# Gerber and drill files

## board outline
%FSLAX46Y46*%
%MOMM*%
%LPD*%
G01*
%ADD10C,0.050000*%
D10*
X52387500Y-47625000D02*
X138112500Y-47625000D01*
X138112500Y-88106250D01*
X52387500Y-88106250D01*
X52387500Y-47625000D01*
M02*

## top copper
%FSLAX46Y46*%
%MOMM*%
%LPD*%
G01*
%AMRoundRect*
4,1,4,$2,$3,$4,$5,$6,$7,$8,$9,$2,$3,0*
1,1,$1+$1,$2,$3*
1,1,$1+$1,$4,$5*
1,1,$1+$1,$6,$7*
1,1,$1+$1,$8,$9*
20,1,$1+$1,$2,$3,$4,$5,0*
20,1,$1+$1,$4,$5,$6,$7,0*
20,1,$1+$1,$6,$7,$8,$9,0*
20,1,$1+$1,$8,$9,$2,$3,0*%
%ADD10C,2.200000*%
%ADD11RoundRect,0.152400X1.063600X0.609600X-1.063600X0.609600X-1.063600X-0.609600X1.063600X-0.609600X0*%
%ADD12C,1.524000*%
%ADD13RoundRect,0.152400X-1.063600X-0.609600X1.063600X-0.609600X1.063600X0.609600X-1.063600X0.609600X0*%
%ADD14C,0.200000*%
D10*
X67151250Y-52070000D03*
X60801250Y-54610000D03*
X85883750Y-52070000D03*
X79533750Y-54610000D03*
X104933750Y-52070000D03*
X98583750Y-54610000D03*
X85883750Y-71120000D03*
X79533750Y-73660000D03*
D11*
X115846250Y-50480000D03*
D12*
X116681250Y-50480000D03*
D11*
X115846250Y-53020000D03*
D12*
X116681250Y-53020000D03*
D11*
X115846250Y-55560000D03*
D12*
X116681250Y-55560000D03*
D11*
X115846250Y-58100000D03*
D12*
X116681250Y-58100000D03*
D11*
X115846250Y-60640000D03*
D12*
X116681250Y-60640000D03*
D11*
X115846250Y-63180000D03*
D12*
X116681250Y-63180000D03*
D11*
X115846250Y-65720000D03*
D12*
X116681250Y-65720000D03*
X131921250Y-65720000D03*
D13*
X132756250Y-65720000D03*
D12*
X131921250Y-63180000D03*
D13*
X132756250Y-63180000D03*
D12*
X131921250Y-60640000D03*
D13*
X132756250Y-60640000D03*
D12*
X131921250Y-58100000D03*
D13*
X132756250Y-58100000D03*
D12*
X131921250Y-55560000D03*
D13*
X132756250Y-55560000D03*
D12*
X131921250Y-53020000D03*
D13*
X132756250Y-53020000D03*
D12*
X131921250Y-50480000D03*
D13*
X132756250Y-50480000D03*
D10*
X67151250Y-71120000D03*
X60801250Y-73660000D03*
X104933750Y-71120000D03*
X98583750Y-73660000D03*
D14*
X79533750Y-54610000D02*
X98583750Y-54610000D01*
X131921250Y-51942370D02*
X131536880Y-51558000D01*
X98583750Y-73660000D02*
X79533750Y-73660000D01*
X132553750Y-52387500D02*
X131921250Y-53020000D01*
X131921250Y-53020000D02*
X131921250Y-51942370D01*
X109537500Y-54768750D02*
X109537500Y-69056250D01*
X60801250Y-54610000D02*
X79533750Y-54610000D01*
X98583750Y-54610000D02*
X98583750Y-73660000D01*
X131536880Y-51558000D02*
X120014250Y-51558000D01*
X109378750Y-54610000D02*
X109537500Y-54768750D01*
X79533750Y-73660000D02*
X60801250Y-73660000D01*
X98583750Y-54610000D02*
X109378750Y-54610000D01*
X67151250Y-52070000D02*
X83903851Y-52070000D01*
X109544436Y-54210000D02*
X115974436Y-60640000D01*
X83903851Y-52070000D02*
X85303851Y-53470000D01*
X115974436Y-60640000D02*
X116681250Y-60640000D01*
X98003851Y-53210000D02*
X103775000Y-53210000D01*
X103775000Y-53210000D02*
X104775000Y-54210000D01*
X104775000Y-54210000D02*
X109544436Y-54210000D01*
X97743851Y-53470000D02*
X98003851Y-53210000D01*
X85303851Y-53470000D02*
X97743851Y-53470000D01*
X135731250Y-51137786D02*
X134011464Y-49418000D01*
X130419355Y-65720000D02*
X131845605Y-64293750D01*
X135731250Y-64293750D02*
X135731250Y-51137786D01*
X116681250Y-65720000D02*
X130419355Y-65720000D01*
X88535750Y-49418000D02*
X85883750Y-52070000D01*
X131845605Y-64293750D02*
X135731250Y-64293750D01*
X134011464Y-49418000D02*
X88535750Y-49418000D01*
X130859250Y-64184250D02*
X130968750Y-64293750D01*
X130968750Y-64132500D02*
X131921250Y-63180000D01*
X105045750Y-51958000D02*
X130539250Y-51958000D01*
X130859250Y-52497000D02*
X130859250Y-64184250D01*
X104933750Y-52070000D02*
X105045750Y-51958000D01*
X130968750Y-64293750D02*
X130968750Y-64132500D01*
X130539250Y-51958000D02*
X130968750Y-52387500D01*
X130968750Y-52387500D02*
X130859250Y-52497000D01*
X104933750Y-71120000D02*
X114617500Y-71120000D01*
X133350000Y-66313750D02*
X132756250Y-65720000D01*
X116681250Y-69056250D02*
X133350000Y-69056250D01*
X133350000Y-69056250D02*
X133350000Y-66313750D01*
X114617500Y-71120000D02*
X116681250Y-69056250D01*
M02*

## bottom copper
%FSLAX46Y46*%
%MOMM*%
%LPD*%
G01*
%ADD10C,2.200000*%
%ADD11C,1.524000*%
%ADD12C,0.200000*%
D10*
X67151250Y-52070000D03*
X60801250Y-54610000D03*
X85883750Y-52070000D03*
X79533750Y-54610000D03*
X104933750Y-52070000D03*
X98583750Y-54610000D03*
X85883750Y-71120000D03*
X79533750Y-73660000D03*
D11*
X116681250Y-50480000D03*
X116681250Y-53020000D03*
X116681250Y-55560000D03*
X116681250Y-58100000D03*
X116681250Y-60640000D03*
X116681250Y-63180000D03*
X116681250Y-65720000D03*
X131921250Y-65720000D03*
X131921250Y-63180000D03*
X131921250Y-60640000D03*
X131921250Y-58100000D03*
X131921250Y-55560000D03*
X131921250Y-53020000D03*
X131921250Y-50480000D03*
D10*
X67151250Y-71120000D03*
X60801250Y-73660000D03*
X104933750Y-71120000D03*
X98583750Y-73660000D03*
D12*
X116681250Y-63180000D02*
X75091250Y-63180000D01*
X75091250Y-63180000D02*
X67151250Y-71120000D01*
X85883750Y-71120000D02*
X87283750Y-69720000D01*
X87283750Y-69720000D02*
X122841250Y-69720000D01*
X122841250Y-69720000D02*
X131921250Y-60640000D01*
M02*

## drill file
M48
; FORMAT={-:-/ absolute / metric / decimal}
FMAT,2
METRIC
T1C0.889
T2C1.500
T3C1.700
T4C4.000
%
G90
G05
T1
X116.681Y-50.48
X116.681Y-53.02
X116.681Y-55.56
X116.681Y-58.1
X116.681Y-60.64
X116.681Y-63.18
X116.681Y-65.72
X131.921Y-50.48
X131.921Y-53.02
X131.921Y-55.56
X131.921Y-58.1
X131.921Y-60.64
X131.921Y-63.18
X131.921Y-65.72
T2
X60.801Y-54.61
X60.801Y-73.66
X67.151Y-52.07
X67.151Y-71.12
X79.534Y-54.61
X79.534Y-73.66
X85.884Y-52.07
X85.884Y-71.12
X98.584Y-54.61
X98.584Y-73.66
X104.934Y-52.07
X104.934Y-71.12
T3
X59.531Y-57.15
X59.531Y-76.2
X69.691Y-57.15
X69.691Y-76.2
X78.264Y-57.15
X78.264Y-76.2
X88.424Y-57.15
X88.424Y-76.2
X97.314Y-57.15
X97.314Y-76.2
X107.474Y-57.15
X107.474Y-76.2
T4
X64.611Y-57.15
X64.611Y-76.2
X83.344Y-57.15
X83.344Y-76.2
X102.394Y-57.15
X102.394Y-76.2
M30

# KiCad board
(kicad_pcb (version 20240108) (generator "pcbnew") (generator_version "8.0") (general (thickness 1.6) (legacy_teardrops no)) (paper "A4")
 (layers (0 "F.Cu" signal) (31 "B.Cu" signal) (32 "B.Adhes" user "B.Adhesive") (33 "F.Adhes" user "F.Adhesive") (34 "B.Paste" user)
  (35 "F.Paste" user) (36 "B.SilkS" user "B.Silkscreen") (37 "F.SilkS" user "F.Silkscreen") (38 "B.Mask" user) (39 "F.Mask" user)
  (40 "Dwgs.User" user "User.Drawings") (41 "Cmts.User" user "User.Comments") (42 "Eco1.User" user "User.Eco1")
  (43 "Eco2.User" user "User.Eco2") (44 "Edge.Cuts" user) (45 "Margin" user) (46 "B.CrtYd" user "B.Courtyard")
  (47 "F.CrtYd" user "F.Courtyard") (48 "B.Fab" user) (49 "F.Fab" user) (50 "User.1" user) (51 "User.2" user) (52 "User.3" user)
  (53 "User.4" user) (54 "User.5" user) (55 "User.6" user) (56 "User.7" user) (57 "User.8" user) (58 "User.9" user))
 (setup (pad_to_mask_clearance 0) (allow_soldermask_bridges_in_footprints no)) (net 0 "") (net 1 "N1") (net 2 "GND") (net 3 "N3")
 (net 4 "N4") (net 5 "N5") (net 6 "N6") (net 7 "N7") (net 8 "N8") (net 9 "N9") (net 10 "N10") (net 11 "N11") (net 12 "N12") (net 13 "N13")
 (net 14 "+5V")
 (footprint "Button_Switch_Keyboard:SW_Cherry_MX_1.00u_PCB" (layer "F.Cu") (at 67.15125 52.07)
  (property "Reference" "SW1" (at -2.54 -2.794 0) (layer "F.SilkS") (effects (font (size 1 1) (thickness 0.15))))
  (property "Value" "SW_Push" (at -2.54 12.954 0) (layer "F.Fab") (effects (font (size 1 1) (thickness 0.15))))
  (pad "" np_thru_hole circle (at -7.62 5.08) (size 1.7 1.7) (drill 1.7) (layers "*.Cu" "*.Mask"))
  (pad "" np_thru_hole circle (at -2.54 5.08) (size 4 4) (drill 4) (layers "*.Cu" "*.Mask"))
  (pad "" np_thru_hole circle (at 2.54 5.08) (size 1.7 1.7) (drill 1.7) (layers "*.Cu" "*.Mask"))
  (pad "1" thru_hole circle (at 0 0) (size 2.2 2.2) (drill 1.5) (layers "*.Cu" "*.Mask") (remove_unused_layers no) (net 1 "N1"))
  (pad "2" thru_hole circle (at -6.35 2.54) (size 2.2 2.2) (drill 1.5) (layers "*.Cu" "*.Mask") (remove_unused_layers no) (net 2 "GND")))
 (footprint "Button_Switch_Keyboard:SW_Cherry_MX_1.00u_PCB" (layer "F.Cu") (at 85.88375 52.07)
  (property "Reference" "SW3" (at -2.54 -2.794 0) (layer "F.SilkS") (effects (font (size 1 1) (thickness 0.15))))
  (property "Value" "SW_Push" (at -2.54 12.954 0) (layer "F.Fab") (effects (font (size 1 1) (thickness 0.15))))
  (pad "" np_thru_hole circle (at -7.62 5.08) (size 1.7 1.7) (drill 1.7) (layers "*.Cu" "*.Mask"))
  (pad "" np_thru_hole circle (at -2.54 5.08) (size 4 4) (drill 4) (layers "*.Cu" "*.Mask"))
  (pad "" np_thru_hole circle (at 2.54 5.08) (size 1.7 1.7) (drill 1.7) (layers "*.Cu" "*.Mask"))
  (pad "1" thru_hole circle (at 0 0) (size 2.2 2.2) (drill 1.5) (layers "*.Cu" "*.Mask") (remove_unused_layers no) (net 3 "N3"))
  (pad "2" thru_hole circle (at -6.35 2.54) (size 2.2 2.2) (drill 1.5) (layers "*.Cu" "*.Mask") (remove_unused_layers no) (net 2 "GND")))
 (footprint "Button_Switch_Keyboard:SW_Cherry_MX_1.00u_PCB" (layer "F.Cu") (at 104.93375 52.07)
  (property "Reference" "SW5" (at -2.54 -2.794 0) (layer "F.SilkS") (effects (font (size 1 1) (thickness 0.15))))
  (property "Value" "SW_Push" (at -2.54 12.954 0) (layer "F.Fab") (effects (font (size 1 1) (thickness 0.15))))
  (pad "" np_thru_hole circle (at -7.62 5.08) (size 1.7 1.7) (drill 1.7) (layers "*.Cu" "*.Mask"))
  (pad "" np_thru_hole circle (at -2.54 5.08) (size 4 4) (drill 4) (layers "*.Cu" "*.Mask"))
  (pad "" np_thru_hole circle (at 2.54 5.08) (size 1.7 1.7) (drill 1.7) (layers "*.Cu" "*.Mask"))
  (pad "1" thru_hole circle (at 0 0) (size 2.2 2.2) (drill 1.5) (layers "*.Cu" "*.Mask") (remove_unused_layers no) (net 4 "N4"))
  (pad "2" thru_hole circle (at -6.35 2.54) (size 2.2 2.2) (drill 1.5) (layers "*.Cu" "*.Mask") (remove_unused_layers no) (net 2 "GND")))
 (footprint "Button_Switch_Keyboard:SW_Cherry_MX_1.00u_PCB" (layer "F.Cu") (at 85.88375 71.12)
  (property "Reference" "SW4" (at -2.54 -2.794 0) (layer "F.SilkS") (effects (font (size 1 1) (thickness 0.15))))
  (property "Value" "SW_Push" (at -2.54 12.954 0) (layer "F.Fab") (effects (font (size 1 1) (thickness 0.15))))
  (pad "" np_thru_hole circle (at -7.62 5.08) (size 1.7 1.7) (drill 1.7) (layers "*.Cu" "*.Mask"))
  (pad "" np_thru_hole circle (at -2.54 5.08) (size 4 4) (drill 4) (layers "*.Cu" "*.Mask"))
  (pad "" np_thru_hole circle (at 2.54 5.08) (size 1.7 1.7) (drill 1.7) (layers "*.Cu" "*.Mask"))
  (pad "1" thru_hole circle (at 0 0) (size 2.2 2.2) (drill 1.5) (layers "*.Cu" "*.Mask") (remove_unused_layers no) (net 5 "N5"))
  (pad "2" thru_hole circle (at -6.35 2.54) (size 2.2 2.2) (drill 1.5) (layers "*.Cu" "*.Mask") (remove_unused_layers no) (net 2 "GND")))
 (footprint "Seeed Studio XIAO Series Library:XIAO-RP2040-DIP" (layer "F.Cu") (at 124.30125 58.1)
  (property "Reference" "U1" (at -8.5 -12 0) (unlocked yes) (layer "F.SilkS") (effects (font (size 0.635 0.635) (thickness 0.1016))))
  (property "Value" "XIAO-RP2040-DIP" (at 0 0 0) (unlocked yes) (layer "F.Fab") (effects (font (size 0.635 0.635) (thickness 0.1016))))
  (pad "1" smd roundrect (at -8.455 -7.62 180) (size 2.432 1.524) (layers "F.Cu" "F.Mask") (roundrect_rratio 0.1) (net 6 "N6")
   (thermal_bridge_angle 45))
  (pad "1" thru_hole circle (at -7.62 -7.62 180) (size 1.524 1.524) (drill 0.889) (layers "*.Cu" "*.Mask") (remove_unused_layers no)
   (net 6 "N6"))
  (pad "2" smd roundrect (at -8.455 -5.08 180) (size 2.432 1.524) (layers "F.Cu" "F.Mask") (roundrect_rratio 0.1) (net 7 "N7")
   (thermal_bridge_angle 45))
  (pad "2" thru_hole circle (at -7.62 -5.08 180) (size 1.524 1.524) (drill 0.889) (layers "*.Cu" "*.Mask") (remove_unused_layers no)
   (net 7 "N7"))
  (pad "3" smd roundrect (at -8.455 -2.54 180) (size 2.432 1.524) (layers "F.Cu" "F.Mask") (roundrect_rratio 0.1) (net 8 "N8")
   (thermal_bridge_angle 45))
  (pad "3" thru_hole circle (at -7.62 -2.54 180) (size 1.524 1.524) (drill 0.889) (layers "*.Cu" "*.Mask") (remove_unused_layers no)
   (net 8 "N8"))
  (pad "4" smd roundrect (at -8.455 0 180) (size 2.432 1.524) (layers "F.Cu" "F.Mask") (roundrect_rratio 0.1) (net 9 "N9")
   (thermal_bridge_angle 45))
  (pad "4" thru_hole circle (at -7.62 0 180) (size 1.524 1.524) (drill 0.889) (layers "*.Cu" "*.Mask") (remove_unused_layers no)
   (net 9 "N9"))
  (pad "5" smd roundrect (at -8.455 2.54 180) (size 2.432 1.524) (layers "F.Cu" "F.Mask") (roundrect_rratio 0.1) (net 1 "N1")
   (thermal_bridge_angle 45))
  (pad "5" thru_hole circle (at -7.62 2.54 180) (size 1.524 1.524) (drill 0.889) (layers "*.Cu" "*.Mask") (remove_unused_layers no)
   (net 1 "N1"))
  (pad "6" smd roundrect (at -8.455 5.08 180) (size 2.432 1.524) (layers "F.Cu" "F.Mask") (roundrect_rratio 0.1) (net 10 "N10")
   (thermal_bridge_angle 45))
  (pad "6" thru_hole circle (at -7.62 5.08 180) (size 1.524 1.524) (drill 0.889) (layers "*.Cu" "*.Mask") (remove_unused_layers no)
   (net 10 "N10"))
  (pad "7" smd roundrect (at -8.455 7.62 180) (size 2.432 1.524) (layers "F.Cu" "F.Mask") (roundrect_rratio 0.1) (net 3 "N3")
   (thermal_bridge_angle 45))
  (pad "7" thru_hole circle (at -7.62 7.62 180) (size 1.524 1.524) (drill 0.889) (layers "*.Cu" "*.Mask") (remove_unused_layers no)
   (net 3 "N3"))
  (pad "8" thru_hole circle (at 7.62 7.62) (size 1.524 1.524) (drill 0.889) (layers "*.Cu" "*.Mask") (remove_unused_layers no)
   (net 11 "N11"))
  (pad "8" smd roundrect (at 8.455 7.62) (size 2.432 1.524) (layers "F.Cu" "F.Mask") (roundrect_rratio 0.1) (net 11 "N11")
   (thermal_bridge_angle 45))
  (pad "9" thru_hole circle (at 7.62 5.08) (size 1.524 1.524) (drill 0.889) (layers "*.Cu" "*.Mask") (remove_unused_layers no) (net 4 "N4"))
  (pad "9" smd roundrect (at 8.455 5.08) (size 2.432 1.524) (layers "F.Cu" "F.Mask") (roundrect_rratio 0.1) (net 4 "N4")
   (thermal_bridge_angle 45))
  (pad "10" thru_hole circle (at 7.62 2.54) (size 1.524 1.524) (drill 0.889) (layers "*.Cu" "*.Mask") (remove_unused_layers no) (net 5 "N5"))
  (pad "10" smd roundrect (at 8.455 2.54) (size 2.432 1.524) (layers "F.Cu" "F.Mask") (roundrect_rratio 0.1) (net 5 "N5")
   (thermal_bridge_angle 45))
  (pad "11" thru_hole circle (at 7.62 0) (size 1.524 1.524) (drill 0.889) (layers "*.Cu" "*.Mask") (remove_unused_layers no) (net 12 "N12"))
  (pad "11" smd roundrect (at 8.455 0) (size 2.432 1.524) (layers "F.Cu" "F.Mask") (roundrect_rratio 0.1) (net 12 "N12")
   (thermal_bridge_angle 45))
  (pad "12" thru_hole circle (at 7.62 -2.54) (size 1.524 1.524) (drill 0.889) (layers "*.Cu" "*.Mask") (remove_unused_layers no)
   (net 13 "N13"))
  (pad "12" smd roundrect (at 8.455 -2.54) (size 2.432 1.524) (layers "F.Cu" "F.Mask") (roundrect_rratio 0.1) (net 13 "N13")
   (thermal_bridge_angle 45))
  (pad "13" thru_hole circle (at 7.62 -5.08) (size 1.524 1.524) (drill 0.889) (layers "*.Cu" "*.Mask") (remove_unused_layers no)
   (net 2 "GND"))
  (pad "13" smd roundrect (at 8.455 -5.08) (size 2.432 1.524) (layers "F.Cu" "F.Mask") (roundrect_rratio 0.1) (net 2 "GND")
   (thermal_bridge_angle 45))
  (pad "14" thru_hole circle (at 7.62 -7.62) (size 1.524 1.524) (drill 0.889) (layers "*.Cu" "*.Mask") (remove_unused_layers no)
   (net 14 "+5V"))
  (pad "14" smd roundrect (at 8.455 -7.62) (size 2.432 1.524) (layers "F.Cu" "F.Mask") (roundrect_rratio 0.1) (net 14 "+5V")
   (thermal_bridge_angle 45)))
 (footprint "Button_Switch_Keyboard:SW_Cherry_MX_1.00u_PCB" (layer "F.Cu") (at 67.15125 71.12)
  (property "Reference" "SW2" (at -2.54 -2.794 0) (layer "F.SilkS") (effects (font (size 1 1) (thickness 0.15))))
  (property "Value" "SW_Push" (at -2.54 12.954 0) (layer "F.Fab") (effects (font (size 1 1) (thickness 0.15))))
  (pad "" np_thru_hole circle (at -7.62 5.08) (size 1.7 1.7) (drill 1.7) (layers "*.Cu" "*.Mask"))
  (pad "" np_thru_hole circle (at -2.54 5.08) (size 4 4) (drill 4) (layers "*.Cu" "*.Mask"))
  (pad "" np_thru_hole circle (at 2.54 5.08) (size 1.7 1.7) (drill 1.7) (layers "*.Cu" "*.Mask"))
  (pad "1" thru_hole circle (at 0 0) (size 2.2 2.2) (drill 1.5) (layers "*.Cu" "*.Mask") (remove_unused_layers no) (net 10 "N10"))
  (pad "2" thru_hole circle (at -6.35 2.54) (size 2.2 2.2) (drill 1.5) (layers "*.Cu" "*.Mask") (remove_unused_layers no) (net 2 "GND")))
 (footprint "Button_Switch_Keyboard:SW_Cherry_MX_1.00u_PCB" (layer "F.Cu") (at 104.93375 71.12)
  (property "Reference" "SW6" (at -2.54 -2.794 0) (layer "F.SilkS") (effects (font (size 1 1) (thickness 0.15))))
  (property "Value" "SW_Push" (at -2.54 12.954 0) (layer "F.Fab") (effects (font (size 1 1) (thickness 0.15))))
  (pad "" np_thru_hole circle (at -7.62 5.08) (size 1.7 1.7) (drill 1.7) (layers "*.Cu" "*.Mask"))
  (pad "" np_thru_hole circle (at -2.54 5.08) (size 4 4) (drill 4) (layers "*.Cu" "*.Mask"))
  (pad "" np_thru_hole circle (at 2.54 5.08) (size 1.7 1.7) (drill 1.7) (layers "*.Cu" "*.Mask"))
  (pad "1" thru_hole circle (at 0 0) (size 2.2 2.2) (drill 1.5) (layers "*.Cu" "*.Mask") (remove_unused_layers no) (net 11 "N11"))
  (pad "2" thru_hole circle (at -6.35 2.54) (size 2.2 2.2) (drill 1.5) (layers "*.Cu" "*.Mask") (remove_unused_layers no) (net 2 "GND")))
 (gr_rect (start 52.3875 47.625) (end 138.1125 88.10625) (stroke (width 0.05) (type default)) (fill none) (layer "Edge.Cuts"))
 (segment (start 79.53375 54.61) (end 98.58375 54.61) (width 0.2) (layer "F.Cu") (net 2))
 (segment (start 131.92125 51.94237) (end 131.53688 51.558) (width 0.2) (layer "F.Cu") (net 2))
 (segment (start 98.58375 73.66) (end 79.53375 73.66) (width 0.2) (layer "F.Cu") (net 2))
 (segment (start 132.55375 52.3875) (end 131.92125 53.02) (width 0.2) (layer "F.Cu") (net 2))
 (segment (start 131.92125 53.02) (end 131.92125 51.94237) (width 0.2) (layer "F.Cu") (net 2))
 (segment (start 109.5375 54.76875) (end 109.5375 69.05625) (width 0.2) (layer "F.Cu") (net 2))
 (segment (start 60.80125 54.61) (end 79.53375 54.61) (width 0.2) (layer "F.Cu") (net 2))
 (segment (start 98.58375 54.61) (end 98.58375 73.66) (width 0.2) (layer "F.Cu") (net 2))
 (segment (start 131.53688 51.558) (end 120.01425 51.558) (width 0.2) (layer "F.Cu") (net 2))
 (segment (start 109.37875 54.61) (end 109.5375 54.76875) (width 0.2) (layer "F.Cu") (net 2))
 (segment (start 79.53375 73.66) (end 60.80125 73.66) (width 0.2) (layer "F.Cu") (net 2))
 (segment (start 98.58375 54.61) (end 109.37875 54.61) (width 0.2) (layer "F.Cu") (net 2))
 (segment (start 67.15125 52.07) (end 83.903851 52.07) (width 0.2) (layer "F.Cu") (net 1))
 (segment (start 109.544436 54.21) (end 115.974436 60.64) (width 0.2) (layer "F.Cu") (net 1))
 (segment (start 83.903851 52.07) (end 85.303851 53.47) (width 0.2) (layer "F.Cu") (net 1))
 (segment (start 115.974436 60.64) (end 116.68125 60.64) (width 0.2) (layer "F.Cu") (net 1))
 (segment (start 98.003851 53.21) (end 103.775 53.21) (width 0.2) (layer "F.Cu") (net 1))
 (segment (start 103.775 53.21) (end 104.775 54.21) (width 0.2) (layer "F.Cu") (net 1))
 (segment (start 104.775 54.21) (end 109.544436 54.21) (width 0.2) (layer "F.Cu") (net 1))
 (segment (start 97.743851 53.47) (end 98.003851 53.21) (width 0.2) (layer "F.Cu") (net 1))
 (segment (start 85.303851 53.47) (end 97.743851 53.47) (width 0.2) (layer "F.Cu") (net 1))
 (segment (start 116.68125 63.18) (end 75.09125 63.18) (width 0.2) (layer "B.Cu") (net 10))
 (segment (start 75.09125 63.18) (end 67.15125 71.12) (width 0.2) (layer "B.Cu") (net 10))
 (segment (start 135.73125 51.137786) (end 134.011464 49.418) (width 0.2) (layer "F.Cu") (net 3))
 (segment (start 130.419355 65.72) (end 131.845605 64.29375) (width 0.2) (layer "F.Cu") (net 3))
 (segment (start 135.73125 64.29375) (end 135.73125 51.137786) (width 0.2) (layer "F.Cu") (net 3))
 (segment (start 116.68125 65.72) (end 130.419355 65.72) (width 0.2) (layer "F.Cu") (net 3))
 (segment (start 88.53575 49.418) (end 85.88375 52.07) (width 0.2) (layer "F.Cu") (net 3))
 (segment (start 131.845605 64.29375) (end 135.73125 64.29375) (width 0.2) (layer "F.Cu") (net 3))
 (segment (start 134.011464 49.418) (end 88.53575 49.418) (width 0.2) (layer "F.Cu") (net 3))
 (segment (start 85.88375 71.12) (end 87.28375 69.72) (width 0.2) (layer "B.Cu") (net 5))
 (segment (start 87.28375 69.72) (end 122.84125 69.72) (width 0.2) (layer "B.Cu") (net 5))
 (segment (start 122.84125 69.72) (end 131.92125 60.64) (width 0.2) (layer "B.Cu") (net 5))
 (segment (start 130.85925 64.18425) (end 130.96875 64.29375) (width 0.2) (layer "F.Cu") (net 4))
 (segment (start 130.96875 64.1325) (end 131.92125 63.18) (width 0.2) (layer "F.Cu") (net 4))
 (segment (start 105.04575 51.958) (end 130.53925 51.958) (width 0.2) (layer "F.Cu") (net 4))
 (segment (start 130.85925 52.497) (end 130.85925 64.18425) (width 0.2) (layer "F.Cu") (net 4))
 (segment (start 104.93375 52.07) (end 105.04575 51.958) (width 0.2) (layer "F.Cu") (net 4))
 (segment (start 130.96875 64.29375) (end 130.96875 64.1325) (width 0.2) (layer "F.Cu") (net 4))
 (segment (start 130.53925 51.958) (end 130.96875 52.3875) (width 0.2) (layer "F.Cu") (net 4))
 (segment (start 130.96875 52.3875) (end 130.85925 52.497) (width 0.2) (layer "F.Cu") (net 4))
 (segment (start 104.93375 71.12) (end 114.6175 71.12) (width 0.2) (layer "F.Cu") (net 11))
 (segment (start 133.35 66.31375) (end 132.75625 65.72) (width 0.2) (layer "F.Cu") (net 11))
 (segment (start 116.68125 69.05625) (end 133.35 69.05625) (width 0.2) (layer "F.Cu") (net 11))
 (segment (start 133.35 69.05625) (end 133.35 66.31375) (width 0.2) (layer "F.Cu") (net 11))
 (segment (start 114.6175 71.12) (end 116.68125 69.05625) (width 0.2) (layer "F.Cu") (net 11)))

